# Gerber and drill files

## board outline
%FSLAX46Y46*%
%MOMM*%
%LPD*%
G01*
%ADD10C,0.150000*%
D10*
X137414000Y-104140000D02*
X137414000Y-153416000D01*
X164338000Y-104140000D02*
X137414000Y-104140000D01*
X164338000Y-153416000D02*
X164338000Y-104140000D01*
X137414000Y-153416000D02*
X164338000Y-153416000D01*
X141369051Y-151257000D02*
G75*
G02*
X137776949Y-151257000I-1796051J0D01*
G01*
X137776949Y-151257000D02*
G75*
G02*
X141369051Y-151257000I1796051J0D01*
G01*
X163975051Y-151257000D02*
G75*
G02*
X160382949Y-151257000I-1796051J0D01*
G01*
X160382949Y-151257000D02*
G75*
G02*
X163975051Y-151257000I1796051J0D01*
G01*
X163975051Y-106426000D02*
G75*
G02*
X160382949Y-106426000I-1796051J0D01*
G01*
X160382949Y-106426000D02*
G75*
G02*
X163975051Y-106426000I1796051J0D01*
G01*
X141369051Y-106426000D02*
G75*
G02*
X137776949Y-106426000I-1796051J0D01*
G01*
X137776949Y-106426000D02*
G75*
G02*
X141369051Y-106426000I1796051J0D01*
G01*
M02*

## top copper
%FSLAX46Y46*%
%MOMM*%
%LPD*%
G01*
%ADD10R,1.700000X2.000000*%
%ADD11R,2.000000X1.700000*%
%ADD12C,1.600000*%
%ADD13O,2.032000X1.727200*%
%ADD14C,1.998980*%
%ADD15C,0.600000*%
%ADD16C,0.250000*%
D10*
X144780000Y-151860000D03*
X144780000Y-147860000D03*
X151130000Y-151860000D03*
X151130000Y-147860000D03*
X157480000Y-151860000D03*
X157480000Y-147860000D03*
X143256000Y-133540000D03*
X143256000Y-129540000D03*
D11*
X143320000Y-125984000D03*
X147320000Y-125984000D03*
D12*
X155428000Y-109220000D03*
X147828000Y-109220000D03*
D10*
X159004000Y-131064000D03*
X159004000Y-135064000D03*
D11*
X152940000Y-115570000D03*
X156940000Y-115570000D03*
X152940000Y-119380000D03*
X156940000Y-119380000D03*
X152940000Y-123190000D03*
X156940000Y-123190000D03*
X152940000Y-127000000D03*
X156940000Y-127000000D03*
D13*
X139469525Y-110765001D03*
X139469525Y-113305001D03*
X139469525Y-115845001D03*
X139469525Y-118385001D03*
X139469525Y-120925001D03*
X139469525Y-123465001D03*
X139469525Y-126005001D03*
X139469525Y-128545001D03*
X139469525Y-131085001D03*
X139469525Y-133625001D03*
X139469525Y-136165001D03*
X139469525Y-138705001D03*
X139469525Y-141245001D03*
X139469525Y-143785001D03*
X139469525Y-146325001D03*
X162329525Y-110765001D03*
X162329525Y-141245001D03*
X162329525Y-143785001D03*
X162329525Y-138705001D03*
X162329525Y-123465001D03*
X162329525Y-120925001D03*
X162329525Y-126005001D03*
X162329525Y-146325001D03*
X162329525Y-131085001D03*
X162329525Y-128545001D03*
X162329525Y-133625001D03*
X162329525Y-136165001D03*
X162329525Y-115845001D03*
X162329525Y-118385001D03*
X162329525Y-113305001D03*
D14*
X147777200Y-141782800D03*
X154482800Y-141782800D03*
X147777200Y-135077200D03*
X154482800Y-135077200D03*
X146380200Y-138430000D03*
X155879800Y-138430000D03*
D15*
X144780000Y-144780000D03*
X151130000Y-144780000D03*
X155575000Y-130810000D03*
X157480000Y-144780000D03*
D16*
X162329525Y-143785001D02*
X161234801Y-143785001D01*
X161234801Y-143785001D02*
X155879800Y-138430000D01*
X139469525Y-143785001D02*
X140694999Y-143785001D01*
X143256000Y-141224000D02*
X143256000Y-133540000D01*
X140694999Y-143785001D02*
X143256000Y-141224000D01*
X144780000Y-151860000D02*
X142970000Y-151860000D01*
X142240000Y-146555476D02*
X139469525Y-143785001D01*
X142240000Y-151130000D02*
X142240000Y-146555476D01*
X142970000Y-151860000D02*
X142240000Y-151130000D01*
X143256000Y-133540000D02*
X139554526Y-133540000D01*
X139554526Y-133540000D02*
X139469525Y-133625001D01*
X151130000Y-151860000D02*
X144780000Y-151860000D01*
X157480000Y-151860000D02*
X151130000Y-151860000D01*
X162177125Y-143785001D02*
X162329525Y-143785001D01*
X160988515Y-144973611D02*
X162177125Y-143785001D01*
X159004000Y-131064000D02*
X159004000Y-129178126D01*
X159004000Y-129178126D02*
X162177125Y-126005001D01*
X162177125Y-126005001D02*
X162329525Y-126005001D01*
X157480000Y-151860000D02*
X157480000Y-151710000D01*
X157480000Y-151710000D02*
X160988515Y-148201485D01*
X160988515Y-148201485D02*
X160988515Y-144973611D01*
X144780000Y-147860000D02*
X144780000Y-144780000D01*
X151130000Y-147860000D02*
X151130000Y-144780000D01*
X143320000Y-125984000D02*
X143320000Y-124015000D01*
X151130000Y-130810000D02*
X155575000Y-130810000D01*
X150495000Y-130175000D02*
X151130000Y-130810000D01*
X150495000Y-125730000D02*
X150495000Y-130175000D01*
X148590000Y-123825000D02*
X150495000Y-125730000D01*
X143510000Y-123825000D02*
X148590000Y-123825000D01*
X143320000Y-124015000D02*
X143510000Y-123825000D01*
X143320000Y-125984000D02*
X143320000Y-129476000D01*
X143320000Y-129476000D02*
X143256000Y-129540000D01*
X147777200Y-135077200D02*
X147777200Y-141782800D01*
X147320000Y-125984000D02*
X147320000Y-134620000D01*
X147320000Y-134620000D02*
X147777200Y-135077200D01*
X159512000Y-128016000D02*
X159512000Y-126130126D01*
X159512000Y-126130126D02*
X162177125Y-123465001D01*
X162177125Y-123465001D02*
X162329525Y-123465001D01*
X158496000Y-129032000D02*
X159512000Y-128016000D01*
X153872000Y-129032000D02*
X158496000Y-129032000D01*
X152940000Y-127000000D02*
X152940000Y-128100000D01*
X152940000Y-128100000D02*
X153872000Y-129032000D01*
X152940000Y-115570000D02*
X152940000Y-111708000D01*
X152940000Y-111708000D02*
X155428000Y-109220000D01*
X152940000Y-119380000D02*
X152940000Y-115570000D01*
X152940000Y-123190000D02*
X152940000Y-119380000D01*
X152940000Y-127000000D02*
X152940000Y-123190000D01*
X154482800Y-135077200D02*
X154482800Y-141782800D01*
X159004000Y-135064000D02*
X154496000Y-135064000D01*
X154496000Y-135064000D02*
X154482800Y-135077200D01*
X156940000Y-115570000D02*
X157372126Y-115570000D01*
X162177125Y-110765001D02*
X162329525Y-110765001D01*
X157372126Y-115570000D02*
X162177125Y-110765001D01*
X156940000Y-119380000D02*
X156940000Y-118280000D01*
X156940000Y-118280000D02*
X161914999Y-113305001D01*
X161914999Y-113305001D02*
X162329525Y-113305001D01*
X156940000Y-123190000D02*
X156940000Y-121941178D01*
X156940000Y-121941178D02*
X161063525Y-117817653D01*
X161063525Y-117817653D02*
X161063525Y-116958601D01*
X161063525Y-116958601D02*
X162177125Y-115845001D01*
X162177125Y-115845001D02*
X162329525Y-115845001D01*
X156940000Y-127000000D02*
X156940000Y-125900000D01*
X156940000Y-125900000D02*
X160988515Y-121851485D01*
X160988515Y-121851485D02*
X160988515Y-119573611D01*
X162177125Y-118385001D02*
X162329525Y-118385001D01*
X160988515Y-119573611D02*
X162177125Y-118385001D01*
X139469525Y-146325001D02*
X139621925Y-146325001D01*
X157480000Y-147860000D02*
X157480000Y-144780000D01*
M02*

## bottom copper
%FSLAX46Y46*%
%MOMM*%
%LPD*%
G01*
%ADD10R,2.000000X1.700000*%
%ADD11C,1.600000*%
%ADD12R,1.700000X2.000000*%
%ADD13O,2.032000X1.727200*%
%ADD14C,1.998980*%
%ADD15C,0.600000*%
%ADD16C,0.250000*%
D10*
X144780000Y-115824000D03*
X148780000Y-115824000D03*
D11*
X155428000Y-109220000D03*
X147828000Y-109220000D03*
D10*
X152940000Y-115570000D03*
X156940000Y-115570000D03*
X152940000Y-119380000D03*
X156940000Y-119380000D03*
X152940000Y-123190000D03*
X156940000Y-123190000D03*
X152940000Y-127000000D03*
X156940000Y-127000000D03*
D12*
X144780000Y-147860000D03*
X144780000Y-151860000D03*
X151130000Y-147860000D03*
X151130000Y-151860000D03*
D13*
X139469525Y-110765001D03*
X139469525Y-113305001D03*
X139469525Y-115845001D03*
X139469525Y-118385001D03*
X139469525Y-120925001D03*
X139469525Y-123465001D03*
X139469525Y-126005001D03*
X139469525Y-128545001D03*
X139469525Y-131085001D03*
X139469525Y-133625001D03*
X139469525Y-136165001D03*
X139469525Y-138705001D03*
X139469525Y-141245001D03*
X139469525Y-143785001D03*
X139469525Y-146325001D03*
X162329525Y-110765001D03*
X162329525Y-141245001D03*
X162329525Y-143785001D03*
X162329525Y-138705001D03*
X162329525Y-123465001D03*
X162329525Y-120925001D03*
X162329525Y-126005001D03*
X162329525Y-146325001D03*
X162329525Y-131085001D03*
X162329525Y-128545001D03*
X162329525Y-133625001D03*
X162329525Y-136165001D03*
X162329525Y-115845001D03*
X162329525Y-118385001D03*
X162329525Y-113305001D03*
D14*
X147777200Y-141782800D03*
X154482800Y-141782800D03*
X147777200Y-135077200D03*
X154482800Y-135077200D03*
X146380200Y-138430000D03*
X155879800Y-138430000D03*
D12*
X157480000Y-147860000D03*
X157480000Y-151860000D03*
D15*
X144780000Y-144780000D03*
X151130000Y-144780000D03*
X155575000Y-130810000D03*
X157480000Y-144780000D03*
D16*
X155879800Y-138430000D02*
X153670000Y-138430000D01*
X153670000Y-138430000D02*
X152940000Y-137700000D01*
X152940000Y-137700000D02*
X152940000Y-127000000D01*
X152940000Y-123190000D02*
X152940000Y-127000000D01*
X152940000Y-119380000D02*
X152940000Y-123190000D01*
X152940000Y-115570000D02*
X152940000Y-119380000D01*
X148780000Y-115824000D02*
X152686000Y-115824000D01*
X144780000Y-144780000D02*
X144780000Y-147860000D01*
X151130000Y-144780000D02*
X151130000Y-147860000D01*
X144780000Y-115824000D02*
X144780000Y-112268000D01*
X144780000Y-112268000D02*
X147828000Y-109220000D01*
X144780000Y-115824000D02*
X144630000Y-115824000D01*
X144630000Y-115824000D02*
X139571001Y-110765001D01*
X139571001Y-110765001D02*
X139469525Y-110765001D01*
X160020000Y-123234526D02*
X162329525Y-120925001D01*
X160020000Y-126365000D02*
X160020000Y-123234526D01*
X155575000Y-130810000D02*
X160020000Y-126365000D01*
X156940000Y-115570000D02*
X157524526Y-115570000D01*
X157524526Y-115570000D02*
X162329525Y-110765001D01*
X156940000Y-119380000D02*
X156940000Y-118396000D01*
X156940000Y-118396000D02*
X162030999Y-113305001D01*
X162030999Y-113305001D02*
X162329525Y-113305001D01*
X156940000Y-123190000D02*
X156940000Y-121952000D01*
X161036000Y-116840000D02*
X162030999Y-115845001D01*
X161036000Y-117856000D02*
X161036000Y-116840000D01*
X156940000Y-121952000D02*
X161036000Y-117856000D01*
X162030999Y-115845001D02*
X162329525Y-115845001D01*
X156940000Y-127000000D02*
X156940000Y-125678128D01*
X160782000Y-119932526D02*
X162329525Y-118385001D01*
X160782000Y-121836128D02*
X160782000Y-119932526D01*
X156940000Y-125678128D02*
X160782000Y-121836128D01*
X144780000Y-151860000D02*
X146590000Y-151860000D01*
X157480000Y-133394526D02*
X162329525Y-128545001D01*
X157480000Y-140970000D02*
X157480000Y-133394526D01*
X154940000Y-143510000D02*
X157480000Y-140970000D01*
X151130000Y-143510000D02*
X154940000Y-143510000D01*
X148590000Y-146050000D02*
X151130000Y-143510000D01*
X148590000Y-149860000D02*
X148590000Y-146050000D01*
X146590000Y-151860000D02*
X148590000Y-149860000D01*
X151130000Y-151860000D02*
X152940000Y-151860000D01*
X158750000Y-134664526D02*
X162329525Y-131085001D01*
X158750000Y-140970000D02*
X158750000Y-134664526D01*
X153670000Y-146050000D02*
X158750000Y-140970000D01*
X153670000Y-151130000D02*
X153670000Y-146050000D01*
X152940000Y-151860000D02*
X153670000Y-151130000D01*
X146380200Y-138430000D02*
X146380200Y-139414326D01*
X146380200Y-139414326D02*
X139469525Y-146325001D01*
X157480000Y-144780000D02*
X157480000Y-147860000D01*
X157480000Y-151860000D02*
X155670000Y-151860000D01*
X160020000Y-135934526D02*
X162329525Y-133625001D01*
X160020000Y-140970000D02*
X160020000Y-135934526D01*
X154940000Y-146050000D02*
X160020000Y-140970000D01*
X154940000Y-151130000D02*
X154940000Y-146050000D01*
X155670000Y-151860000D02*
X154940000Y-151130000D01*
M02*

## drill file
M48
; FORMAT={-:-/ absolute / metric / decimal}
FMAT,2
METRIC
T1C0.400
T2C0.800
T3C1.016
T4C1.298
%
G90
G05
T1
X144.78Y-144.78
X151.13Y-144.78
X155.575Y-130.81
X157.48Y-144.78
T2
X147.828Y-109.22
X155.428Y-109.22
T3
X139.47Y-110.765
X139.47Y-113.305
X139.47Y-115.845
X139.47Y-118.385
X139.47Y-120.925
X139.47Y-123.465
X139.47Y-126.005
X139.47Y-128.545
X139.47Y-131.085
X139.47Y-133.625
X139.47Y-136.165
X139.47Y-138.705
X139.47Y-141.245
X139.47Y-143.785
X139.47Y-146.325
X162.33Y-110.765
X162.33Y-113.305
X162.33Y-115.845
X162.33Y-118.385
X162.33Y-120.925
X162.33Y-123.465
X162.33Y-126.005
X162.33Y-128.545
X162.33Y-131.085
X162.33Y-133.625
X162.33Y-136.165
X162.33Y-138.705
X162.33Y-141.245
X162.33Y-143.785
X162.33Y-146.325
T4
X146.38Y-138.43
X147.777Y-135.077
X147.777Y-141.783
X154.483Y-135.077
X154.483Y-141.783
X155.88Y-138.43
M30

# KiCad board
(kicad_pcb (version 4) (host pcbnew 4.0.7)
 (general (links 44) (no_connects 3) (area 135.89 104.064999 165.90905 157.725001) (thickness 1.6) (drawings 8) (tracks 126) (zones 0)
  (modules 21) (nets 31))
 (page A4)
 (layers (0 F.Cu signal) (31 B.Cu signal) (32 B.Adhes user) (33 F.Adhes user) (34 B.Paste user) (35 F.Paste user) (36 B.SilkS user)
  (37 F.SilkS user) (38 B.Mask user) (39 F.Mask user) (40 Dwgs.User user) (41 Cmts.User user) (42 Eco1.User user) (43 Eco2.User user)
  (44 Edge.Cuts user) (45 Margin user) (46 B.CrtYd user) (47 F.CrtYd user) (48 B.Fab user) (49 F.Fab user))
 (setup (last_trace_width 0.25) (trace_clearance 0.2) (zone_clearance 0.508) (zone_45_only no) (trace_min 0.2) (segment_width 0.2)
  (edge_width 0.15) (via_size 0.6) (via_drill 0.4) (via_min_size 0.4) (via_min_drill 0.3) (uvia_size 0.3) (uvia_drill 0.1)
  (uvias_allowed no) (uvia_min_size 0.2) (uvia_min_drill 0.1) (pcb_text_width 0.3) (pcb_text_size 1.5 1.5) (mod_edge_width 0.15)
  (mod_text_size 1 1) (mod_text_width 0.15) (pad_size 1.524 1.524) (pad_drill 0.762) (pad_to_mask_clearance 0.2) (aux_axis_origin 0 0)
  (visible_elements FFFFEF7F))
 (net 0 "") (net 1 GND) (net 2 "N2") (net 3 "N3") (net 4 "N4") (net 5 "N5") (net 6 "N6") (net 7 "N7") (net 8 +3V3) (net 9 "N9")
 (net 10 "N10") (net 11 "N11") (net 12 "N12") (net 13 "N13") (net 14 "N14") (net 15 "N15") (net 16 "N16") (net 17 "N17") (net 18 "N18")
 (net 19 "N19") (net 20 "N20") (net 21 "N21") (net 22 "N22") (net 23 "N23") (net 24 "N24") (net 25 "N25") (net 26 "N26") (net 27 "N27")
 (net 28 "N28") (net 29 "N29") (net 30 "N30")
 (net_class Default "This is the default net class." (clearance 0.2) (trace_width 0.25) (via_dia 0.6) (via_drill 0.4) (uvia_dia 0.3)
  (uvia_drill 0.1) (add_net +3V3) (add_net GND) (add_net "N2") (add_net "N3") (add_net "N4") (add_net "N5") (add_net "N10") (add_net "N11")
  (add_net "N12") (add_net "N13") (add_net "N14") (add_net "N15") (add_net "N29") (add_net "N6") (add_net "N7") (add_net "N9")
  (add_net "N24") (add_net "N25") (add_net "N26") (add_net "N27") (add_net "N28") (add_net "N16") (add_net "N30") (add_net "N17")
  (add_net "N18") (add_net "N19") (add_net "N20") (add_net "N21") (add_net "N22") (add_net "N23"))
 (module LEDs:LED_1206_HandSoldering (layer F.Cu) (at 144.78 149.86 90)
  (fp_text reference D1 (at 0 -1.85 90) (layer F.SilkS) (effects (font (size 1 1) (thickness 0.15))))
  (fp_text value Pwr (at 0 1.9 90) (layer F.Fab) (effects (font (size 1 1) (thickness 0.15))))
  (pad 1 smd rect (at -2 0 90) (size 2 1.7) (layers F.Cu F.Paste F.Mask) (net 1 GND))
  (pad 2 smd rect (at 2 0 90) (size 2 1.7) (layers F.Cu F.Paste F.Mask) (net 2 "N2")))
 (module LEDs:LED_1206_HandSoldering (layer F.Cu) (at 151.13 149.86 90)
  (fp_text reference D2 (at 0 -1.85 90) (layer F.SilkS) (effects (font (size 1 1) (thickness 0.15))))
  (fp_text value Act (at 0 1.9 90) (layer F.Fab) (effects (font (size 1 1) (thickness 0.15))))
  (pad 1 smd rect (at -2 0 90) (size 2 1.7) (layers F.Cu F.Paste F.Mask) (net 1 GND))
  (pad 2 smd rect (at 2 0 90) (size 2 1.7) (layers F.Cu F.Paste F.Mask) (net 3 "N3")))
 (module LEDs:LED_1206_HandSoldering (layer F.Cu) (at 157.48 149.86 90)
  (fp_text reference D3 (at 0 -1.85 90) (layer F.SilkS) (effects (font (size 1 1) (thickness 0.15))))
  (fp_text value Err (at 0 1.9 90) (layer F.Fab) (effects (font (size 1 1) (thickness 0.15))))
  (pad 1 smd rect (at -2 0 90) (size 2 1.7) (layers F.Cu F.Paste F.Mask) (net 1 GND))
  (pad 2 smd rect (at 2 0 90) (size 2 1.7) (layers F.Cu F.Paste F.Mask) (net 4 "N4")))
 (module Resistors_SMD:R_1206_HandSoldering (layer B.Cu) (at 146.78 115.824)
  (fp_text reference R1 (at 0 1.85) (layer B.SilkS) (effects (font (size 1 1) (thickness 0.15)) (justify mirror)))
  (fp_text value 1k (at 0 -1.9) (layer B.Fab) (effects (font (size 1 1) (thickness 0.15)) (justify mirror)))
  (pad 1 smd rect (at -2 0) (size 2 1.7) (layers B.Cu B.Paste B.Mask) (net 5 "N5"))
  (pad 2 smd rect (at 2 0) (size 2 1.7) (layers B.Cu B.Paste B.Mask) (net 1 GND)))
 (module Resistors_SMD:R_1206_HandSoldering (layer F.Cu) (at 143.256 131.54 90)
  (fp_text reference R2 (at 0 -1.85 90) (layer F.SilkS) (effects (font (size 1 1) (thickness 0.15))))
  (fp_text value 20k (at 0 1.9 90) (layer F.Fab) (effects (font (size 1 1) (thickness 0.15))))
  (pad 1 smd rect (at -2 0 90) (size 2 1.7) (layers F.Cu F.Paste F.Mask) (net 1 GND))
  (pad 2 smd rect (at 2 0 90) (size 2 1.7) (layers F.Cu F.Paste F.Mask) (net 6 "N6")))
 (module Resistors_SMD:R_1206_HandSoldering (layer F.Cu) (at 145.32 125.984)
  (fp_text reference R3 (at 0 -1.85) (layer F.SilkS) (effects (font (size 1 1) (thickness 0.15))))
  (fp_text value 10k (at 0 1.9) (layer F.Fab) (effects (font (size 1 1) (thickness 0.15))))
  (pad 1 smd rect (at -2 0) (size 2 1.7) (layers F.Cu F.Paste F.Mask) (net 6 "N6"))
  (pad 2 smd rect (at 2 0) (size 2 1.7) (layers F.Cu F.Paste F.Mask) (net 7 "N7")))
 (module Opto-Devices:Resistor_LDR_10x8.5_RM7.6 (layer F.Cu) (at 155.428 109.22 180)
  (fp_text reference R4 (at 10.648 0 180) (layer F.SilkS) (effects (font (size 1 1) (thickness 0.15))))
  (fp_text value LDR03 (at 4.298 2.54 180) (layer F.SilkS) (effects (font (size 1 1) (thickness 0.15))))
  (pad 1 thru_hole circle (at 0 0 180) (size 1.6 1.6) (drill 0.8) (layers *.Cu *.Mask) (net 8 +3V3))
  (pad 2 thru_hole circle (at 7.6 0 180) (size 1.6 1.6) (drill 0.8) (layers *.Cu *.Mask) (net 5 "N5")))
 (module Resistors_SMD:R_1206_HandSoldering (layer F.Cu) (at 159.004 133.064 270)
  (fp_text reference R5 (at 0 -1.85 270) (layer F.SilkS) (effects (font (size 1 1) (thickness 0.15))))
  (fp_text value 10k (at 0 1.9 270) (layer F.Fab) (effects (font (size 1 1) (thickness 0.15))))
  (pad 1 smd rect (at -2 0 270) (size 2 1.7) (layers F.Cu F.Paste F.Mask) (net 1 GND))
  (pad 2 smd rect (at 2 0 270) (size 2 1.7) (layers F.Cu F.Paste F.Mask) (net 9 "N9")))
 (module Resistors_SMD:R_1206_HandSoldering (layer F.Cu) (at 154.94 115.57)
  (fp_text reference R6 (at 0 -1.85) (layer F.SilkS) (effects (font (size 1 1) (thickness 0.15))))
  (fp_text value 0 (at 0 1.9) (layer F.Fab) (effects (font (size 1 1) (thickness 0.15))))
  (pad 1 smd rect (at -2 0) (size 2 1.7) (layers F.Cu F.Paste F.Mask) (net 8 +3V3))
  (pad 2 smd rect (at 2 0) (size 2 1.7) (layers F.Cu F.Paste F.Mask) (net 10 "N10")))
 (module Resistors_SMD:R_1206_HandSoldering (layer F.Cu) (at 154.94 119.38)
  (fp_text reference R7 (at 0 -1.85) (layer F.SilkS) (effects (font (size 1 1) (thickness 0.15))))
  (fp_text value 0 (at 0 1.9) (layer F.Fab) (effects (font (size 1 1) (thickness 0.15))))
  (pad 1 smd rect (at -2 0) (size 2 1.7) (layers F.Cu F.Paste F.Mask) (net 8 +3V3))
  (pad 2 smd rect (at 2 0) (size 2 1.7) (layers F.Cu F.Paste F.Mask) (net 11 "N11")))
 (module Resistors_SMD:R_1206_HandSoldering (layer F.Cu) (at 154.94 123.19)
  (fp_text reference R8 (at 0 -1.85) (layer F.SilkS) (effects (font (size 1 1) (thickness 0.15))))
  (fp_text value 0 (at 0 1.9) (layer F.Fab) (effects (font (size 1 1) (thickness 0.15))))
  (pad 1 smd rect (at -2 0) (size 2 1.7) (layers F.Cu F.Paste F.Mask) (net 8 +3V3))
  (pad 2 smd rect (at 2 0) (size 2 1.7) (layers F.Cu F.Paste F.Mask) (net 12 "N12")))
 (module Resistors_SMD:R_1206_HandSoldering (layer F.Cu) (at 154.94 127)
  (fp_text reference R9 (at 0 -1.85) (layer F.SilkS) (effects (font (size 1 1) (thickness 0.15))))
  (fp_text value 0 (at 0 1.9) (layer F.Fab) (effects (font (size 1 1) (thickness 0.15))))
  (pad 1 smd rect (at -2 0) (size 2 1.7) (layers F.Cu F.Paste F.Mask) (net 8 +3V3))
  (pad 2 smd rect (at 2 0) (size 2 1.7) (layers F.Cu F.Paste F.Mask) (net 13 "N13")))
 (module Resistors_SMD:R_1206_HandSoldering (layer B.Cu) (at 154.94 115.57)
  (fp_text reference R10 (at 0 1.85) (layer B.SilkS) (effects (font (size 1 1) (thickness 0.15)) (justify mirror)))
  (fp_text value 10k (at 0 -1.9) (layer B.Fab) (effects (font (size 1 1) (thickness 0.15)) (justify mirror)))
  (pad 1 smd rect (at -2 0) (size 2 1.7) (layers B.Cu B.Paste B.Mask) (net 1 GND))
  (pad 2 smd rect (at 2 0) (size 2 1.7) (layers B.Cu B.Paste B.Mask) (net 10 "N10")))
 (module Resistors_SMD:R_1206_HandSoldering (layer B.Cu) (at 154.94 119.38)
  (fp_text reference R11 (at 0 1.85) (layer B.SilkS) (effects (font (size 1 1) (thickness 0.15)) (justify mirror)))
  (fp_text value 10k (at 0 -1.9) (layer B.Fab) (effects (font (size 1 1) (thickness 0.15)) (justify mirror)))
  (pad 1 smd rect (at -2 0) (size 2 1.7) (layers B.Cu B.Paste B.Mask) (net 1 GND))
  (pad 2 smd rect (at 2 0) (size 2 1.7) (layers B.Cu B.Paste B.Mask) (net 11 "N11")))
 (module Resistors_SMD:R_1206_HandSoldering (layer B.Cu) (at 154.94 123.19)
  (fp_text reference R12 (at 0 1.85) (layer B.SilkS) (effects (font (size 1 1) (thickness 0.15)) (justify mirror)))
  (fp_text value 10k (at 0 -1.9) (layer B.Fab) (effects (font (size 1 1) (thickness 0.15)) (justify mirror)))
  (pad 1 smd rect (at -2 0) (size 2 1.7) (layers B.Cu B.Paste B.Mask) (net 1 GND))
  (pad 2 smd rect (at 2 0) (size 2 1.7) (layers B.Cu B.Paste B.Mask) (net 12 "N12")))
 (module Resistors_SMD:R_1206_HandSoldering (layer B.Cu) (at 154.94 127)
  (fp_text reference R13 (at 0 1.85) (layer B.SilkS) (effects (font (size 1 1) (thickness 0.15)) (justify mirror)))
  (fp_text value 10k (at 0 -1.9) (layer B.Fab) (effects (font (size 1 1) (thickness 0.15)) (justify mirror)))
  (pad 1 smd rect (at -2 0) (size 2 1.7) (layers B.Cu B.Paste B.Mask) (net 1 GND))
  (pad 2 smd rect (at 2 0) (size 2 1.7) (layers B.Cu B.Paste B.Mask) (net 13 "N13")))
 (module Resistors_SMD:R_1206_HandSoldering (layer B.Cu) (at 144.78 149.86 270)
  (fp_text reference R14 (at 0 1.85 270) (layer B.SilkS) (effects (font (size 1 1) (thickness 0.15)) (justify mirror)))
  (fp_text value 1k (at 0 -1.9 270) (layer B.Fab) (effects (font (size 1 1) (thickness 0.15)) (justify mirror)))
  (pad 1 smd rect (at -2 0 270) (size 2 1.7) (layers B.Cu B.Paste B.Mask) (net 2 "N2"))
  (pad 2 smd rect (at 2 0 270) (size 2 1.7) (layers B.Cu B.Paste B.Mask) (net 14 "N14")))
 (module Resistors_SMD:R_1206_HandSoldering (layer B.Cu) (at 151.13 149.86 270)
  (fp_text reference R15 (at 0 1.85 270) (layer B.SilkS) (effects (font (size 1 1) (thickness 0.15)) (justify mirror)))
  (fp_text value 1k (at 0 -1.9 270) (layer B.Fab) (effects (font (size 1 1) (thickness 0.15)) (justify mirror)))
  (pad 1 smd rect (at -2 0 270) (size 2 1.7) (layers B.Cu B.Paste B.Mask) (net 3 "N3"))
  (pad 2 smd rect (at 2 0 270) (size 2 1.7) (layers B.Cu B.Paste B.Mask) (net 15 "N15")))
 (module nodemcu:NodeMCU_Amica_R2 (layer F.Cu) (at 139.469525 110.765001)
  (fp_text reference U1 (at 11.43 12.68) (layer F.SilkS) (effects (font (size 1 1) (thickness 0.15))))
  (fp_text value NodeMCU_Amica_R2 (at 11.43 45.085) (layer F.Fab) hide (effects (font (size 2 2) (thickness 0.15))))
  (pad 1 thru_hole oval (at 0 0) (size 2.032 1.7272) (drill 1.016) (layers *.Cu *.Mask F.SilkS) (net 5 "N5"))
  (pad 2 thru_hole oval (at 0 2.54) (size 2.032 1.7272) (drill 1.016) (layers *.Cu *.Mask F.SilkS) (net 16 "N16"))
  (pad 3 thru_hole oval (at 0 5.08) (size 2.032 1.7272) (drill 1.016) (layers *.Cu *.Mask F.SilkS) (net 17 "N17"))
  (pad 4 thru_hole oval (at 0 7.62) (size 2.032 1.7272) (drill 1.016) (layers *.Cu *.Mask F.SilkS) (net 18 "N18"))
  (pad 5 thru_hole oval (at 0 10.16) (size 2.032 1.7272) (drill 1.016) (layers *.Cu *.Mask F.SilkS) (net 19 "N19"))
  (pad 6 thru_hole oval (at 0 12.7) (size 2.032 1.7272) (drill 1.016) (layers *.Cu *.Mask F.SilkS) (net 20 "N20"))
  (pad 7 thru_hole oval (at 0 15.24) (size 2.032 1.7272) (drill 1.016) (layers *.Cu *.Mask F.SilkS) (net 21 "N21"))
  (pad 8 thru_hole oval (at 0 17.78) (size 2.032 1.7272) (drill 1.016) (layers *.Cu *.Mask F.SilkS) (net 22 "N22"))
  (pad 9 thru_hole oval (at 0 20.32) (size 2.032 1.7272) (drill 1.016) (layers *.Cu *.Mask F.SilkS) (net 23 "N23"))
  (pad 10 thru_hole oval (at 0 22.86) (size 2.032 1.7272) (drill 1.016) (layers *.Cu *.Mask F.SilkS) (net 1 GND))
  (pad 11 thru_hole oval (at 0 25.4) (size 2.032 1.7272) (drill 1.016) (layers *.Cu *.Mask F.SilkS) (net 8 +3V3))
  (pad 12 thru_hole oval (at 0 27.94) (size 2.032 1.7272) (drill 1.016) (layers *.Cu *.Mask F.SilkS) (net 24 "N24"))
  (pad 13 thru_hole oval (at 0 30.48) (size 2.032 1.7272) (drill 1.016) (layers *.Cu *.Mask F.SilkS) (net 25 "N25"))
  (pad 14 thru_hole oval (at 0 33.02) (size 2.032 1.7272) (drill 1.016) (layers *.Cu *.Mask F.SilkS) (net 1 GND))
  (pad 15 thru_hole oval (at 0 35.56) (size 2.032 1.7272) (drill 1.016) (layers *.Cu *.Mask F.SilkS) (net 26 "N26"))
  (pad 30 thru_hole oval (at 22.86 0) (size 2.032 1.7272) (drill 1.016) (layers *.Cu *.Mask F.SilkS) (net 10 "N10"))
  (pad 18 thru_hole oval (at 22.86 30.48) (size 2.032 1.7272) (drill 1.016) (layers *.Cu *.Mask F.SilkS) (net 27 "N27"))
  (pad 17 thru_hole oval (at 22.86 33.02) (size 2.032 1.7272) (drill 1.016) (layers *.Cu *.Mask F.SilkS) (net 1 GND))
  (pad 19 thru_hole oval (at 22.86 27.94) (size 2.032 1.7272) (drill 1.016) (layers *.Cu *.Mask F.SilkS) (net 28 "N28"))
  (pad 25 thru_hole oval (at 22.86 12.7) (size 2.032 1.7272) (drill 1.016) (layers *.Cu *.Mask F.SilkS) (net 8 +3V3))
  (pad 26 thru_hole oval (at 22.86 10.16) (size 2.032 1.7272) (drill 1.016) (layers *.Cu *.Mask F.SilkS) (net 6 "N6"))
  (pad 24 thru_hole oval (at 22.86 15.24) (size 2.032 1.7272) (drill 1.016) (layers *.Cu *.Mask F.SilkS) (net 1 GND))
  (pad 16 thru_hole oval (at 22.86 35.56) (size 2.032 1.7272) (drill 1.016) (layers *.Cu *.Mask F.SilkS) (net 8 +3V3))
  (pad 22 thru_hole oval (at 22.86 20.32) (size 2.032 1.7272) (drill 1.016) (layers *.Cu *.Mask F.SilkS) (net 15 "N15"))
  (pad 23 thru_hole oval (at 22.86 17.78) (size 2.032 1.7272) (drill 1.016) (layers *.Cu *.Mask F.SilkS) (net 14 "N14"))
  (pad 21 thru_hole oval (at 22.86 22.86) (size 2.032 1.7272) (drill 1.016) (layers *.Cu *.Mask F.SilkS) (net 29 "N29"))
  (pad 20 thru_hole oval (at 22.86 25.4) (size 2.032 1.7272) (drill 1.016) (layers *.Cu *.Mask F.SilkS) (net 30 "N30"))
  (pad 28 thru_hole oval (at 22.86 5.08) (size 2.032 1.7272) (drill 1.016) (layers *.Cu *.Mask F.SilkS) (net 12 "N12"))
  (pad 27 thru_hole oval (at 22.86 7.62) (size 2.032 1.7272) (drill 1.016) (layers *.Cu *.Mask F.SilkS) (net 13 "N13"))
  (pad 29 thru_hole oval (at 22.86 2.54) (size 2.032 1.7272) (drill 1.016) (layers *.Cu *.Mask F.SilkS) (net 11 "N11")))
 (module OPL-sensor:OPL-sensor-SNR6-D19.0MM (layer F.Cu) (at 151.13 138.43 90)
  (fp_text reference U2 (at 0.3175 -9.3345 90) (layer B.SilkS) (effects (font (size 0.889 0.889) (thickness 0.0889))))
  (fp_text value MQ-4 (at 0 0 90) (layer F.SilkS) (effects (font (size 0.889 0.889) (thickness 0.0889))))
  (pad 1 thru_hole circle (at -3.3528 -3.3528 90) (size 1.99898 1.99898) (drill 1.29794) (layers *.Cu F.Paste F.SilkS F.Mask) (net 7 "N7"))
  (pad 2 thru_hole circle (at -3.3528 3.3528 90) (size 1.99898 1.99898) (drill 1.29794) (layers *.Cu F.Paste F.SilkS F.Mask) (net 9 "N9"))
  (pad 3 thru_hole circle (at 3.3528 -3.3528 90) (size 1.99898 1.99898) (drill 1.29794) (layers *.Cu F.Paste F.SilkS F.Mask) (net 7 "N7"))
  (pad 4 thru_hole circle (at 3.3528 3.3528 90) (size 1.99898 1.99898) (drill 1.29794) (layers *.Cu F.Paste F.SilkS F.Mask) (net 9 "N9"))
  (pad 5 thru_hole circle (at 0 -4.7498 90) (size 1.99898 1.99898) (drill 1.29794) (layers *.Cu F.Paste F.SilkS F.Mask) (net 26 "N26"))
  (pad 6 thru_hole circle (at 0 4.7498 90) (size 1.99898 1.99898) (drill 1.29794) (layers *.Cu F.Paste F.SilkS F.Mask) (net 1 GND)))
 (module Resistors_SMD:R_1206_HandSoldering (layer B.Cu) (at 157.48 149.86 270)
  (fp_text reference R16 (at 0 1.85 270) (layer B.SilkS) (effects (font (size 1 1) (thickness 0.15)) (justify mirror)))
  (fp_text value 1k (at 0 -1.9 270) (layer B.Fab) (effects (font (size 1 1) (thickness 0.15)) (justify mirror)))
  (pad 1 smd rect (at -2 0 270) (size 2 1.7) (layers B.Cu B.Paste B.Mask) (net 4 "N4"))
  (pad 2 smd rect (at 2 0 270) (size 2 1.7) (layers B.Cu B.Paste B.Mask) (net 29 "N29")))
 (gr_line (start 137.414 104.14) (end 137.414 153.416) (angle 90) (layer Edge.Cuts) (width 0.15))
 (gr_line (start 164.338 104.14) (end 137.414 104.14) (angle 90) (layer Edge.Cuts) (width 0.15))
 (gr_line (start 164.338 153.416) (end 164.338 104.14) (angle 90) (layer Edge.Cuts) (width 0.15))
 (gr_line (start 137.414 153.416) (end 164.338 153.416) (angle 90) (layer Edge.Cuts) (width 0.15))
 (gr_circle (center 139.573 151.257) (end 140.843 152.527) (layer Edge.Cuts) (width 0.15))
 (gr_circle (center 162.179 151.257) (end 163.449 152.527) (layer Edge.Cuts) (width 0.15))
 (gr_circle (center 162.179 106.426) (end 163.449 107.696) (layer Edge.Cuts) (width 0.15))
 (gr_circle (center 139.573 106.426) (end 140.843 107.696) (layer Edge.Cuts) (width 0.15))
 (segment (start 162.329525 143.785001) (end 161.234801 143.785001) (width 0.25) (layer F.Cu) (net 1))
 (segment (start 161.234801 143.785001) (end 155.8798 138.43) (width 0.25) (layer F.Cu) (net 1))
 (segment (start 139.469525 143.785001) (end 140.694999 143.785001) (width 0.25) (layer F.Cu) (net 1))
 (segment (start 143.256 141.224) (end 143.256 133.54) (width 0.25) (layer F.Cu) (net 1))
 (segment (start 140.694999 143.785001) (end 143.256 141.224) (width 0.25) (layer F.Cu) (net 1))
 (segment (start 144.78 151.86) (end 142.97 151.86) (width 0.25) (layer F.Cu) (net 1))
 (segment (start 142.24 146.555476) (end 139.469525 143.785001) (width 0.25) (layer F.Cu) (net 1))
 (segment (start 142.24 151.13) (end 142.24 146.555476) (width 0.25) (layer F.Cu) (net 1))
 (segment (start 142.97 151.86) (end 142.24 151.13) (width 0.25) (layer F.Cu) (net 1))
 (segment (start 155.8798 138.43) (end 153.67 138.43) (width 0.25) (layer B.Cu) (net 1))
 (segment (start 153.67 138.43) (end 152.94 137.7) (width 0.25) (layer B.Cu) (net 1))
 (segment (start 152.94 137.7) (end 152.94 127) (width 0.25) (layer B.Cu) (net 1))
 (segment (start 152.94 123.19) (end 152.94 127) (width 0.25) (layer B.Cu) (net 1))
 (segment (start 152.94 119.38) (end 152.94 123.19) (width 0.25) (layer B.Cu) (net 1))
 (segment (start 152.94 115.57) (end 152.94 119.38) (width 0.25) (layer B.Cu) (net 1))
 (segment (start 148.78 115.824) (end 152.686 115.824) (width 0.25) (layer B.Cu) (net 1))
 (segment (start 143.256 133.54) (end 139.554526 133.54) (width 0.25) (layer F.Cu) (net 1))
 (segment (start 139.554526 133.54) (end 139.469525 133.625001) (width 0.25) (layer F.Cu) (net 1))
 (segment (start 151.13 151.86) (end 144.78 151.86) (width 0.25) (layer F.Cu) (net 1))
 (segment (start 157.48 151.86) (end 151.13 151.86) (width 0.25) (layer F.Cu) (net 1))
 (segment (start 162.177125 143.785001) (end 162.329525 143.785001) (width 0.25) (layer F.Cu) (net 1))
 (segment (start 160.988515 144.973611) (end 162.177125 143.785001) (width 0.25) (layer F.Cu) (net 1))
 (segment (start 159.004 131.064) (end 159.004 129.178126) (width 0.25) (layer F.Cu) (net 1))
 (segment (start 159.004 129.178126) (end 162.177125 126.005001) (width 0.25) (layer F.Cu) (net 1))
 (segment (start 162.177125 126.005001) (end 162.329525 126.005001) (width 0.25) (layer F.Cu) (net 1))
 (segment (start 157.48 151.86) (end 157.48 151.71) (width 0.25) (layer F.Cu) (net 1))
 (segment (start 157.48 151.71) (end 160.988515 148.201485) (width 0.25) (layer F.Cu) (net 1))
 (segment (start 160.988515 148.201485) (end 160.988515 144.973611) (width 0.25) (layer F.Cu) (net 1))
 (segment (start 144.78 147.86) (end 144.78 144.78) (width 0.25) (layer F.Cu) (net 2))
 (segment (start 144.78 144.78) (end 144.78 147.86) (width 0.25) (layer B.Cu) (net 2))
 (via (at 144.78 144.78) (size 0.6) (drill 0.4) (layers F.Cu B.Cu) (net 2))
 (segment (start 151.13 147.86) (end 151.13 144.78) (width 0.25) (layer F.Cu) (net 3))
 (segment (start 151.13 144.78) (end 151.13 147.86) (width 0.25) (layer B.Cu) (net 3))
 (via (at 151.13 144.78) (size 0.6) (drill 0.4) (layers F.Cu B.Cu) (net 3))
 (segment (start 144.78 115.824) (end 144.78 112.268) (width 0.25) (layer B.Cu) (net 5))
 (segment (start 144.78 112.268) (end 147.828 109.22) (width 0.25) (layer B.Cu) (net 5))
 (segment (start 144.78 115.824) (end 144.63 115.824) (width 0.25) (layer B.Cu) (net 5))
 (segment (start 144.63 115.824) (end 139.571001 110.765001) (width 0.25) (layer B.Cu) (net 5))
 (segment (start 139.571001 110.765001) (end 139.469525 110.765001) (width 0.25) (layer B.Cu) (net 5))
 (segment (start 143.32 125.984) (end 143.32 124.015) (width 0.25) (layer F.Cu) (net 6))
 (segment (start 160.02 123.234526) (end 162.329525 120.925001) (width 0.25) (layer B.Cu) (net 6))
 (segment (start 160.02 126.365) (end 160.02 123.234526) (width 0.25) (layer B.Cu) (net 6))
 (segment (start 155.575 130.81) (end 160.02 126.365) (width 0.25) (layer B.Cu) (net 6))
 (via (at 155.575 130.81) (size 0.6) (drill 0.4) (layers F.Cu B.Cu) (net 6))
 (segment (start 151.13 130.81) (end 155.575 130.81) (width 0.25) (layer F.Cu) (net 6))
 (segment (start 150.495 130.175) (end 151.13 130.81) (width 0.25) (layer F.Cu) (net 6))
 (segment (start 150.495 125.73) (end 150.495 130.175) (width 0.25) (layer F.Cu) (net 6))
 (segment (start 148.59 123.825) (end 150.495 125.73) (width 0.25) (layer F.Cu) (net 6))
 (segment (start 143.51 123.825) (end 148.59 123.825) (width 0.25) (layer F.Cu) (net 6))
 (segment (start 143.32 124.015) (end 143.51 123.825) (width 0.25) (layer F.Cu) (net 6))
 (segment (start 143.32 125.984) (end 143.32 129.476) (width 0.25) (layer F.Cu) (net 6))
 (segment (start 143.32 129.476) (end 143.256 129.54) (width 0.25) (layer F.Cu) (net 6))
 (segment (start 147.7772 135.0772) (end 147.7772 141.7828) (width 0.25) (layer F.Cu) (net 7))
 (segment (start 147.32 125.984) (end 147.32 134.62) (width 0.25) (layer F.Cu) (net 7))
 (segment (start 147.32 134.62) (end 147.7772 135.0772) (width 0.25) (layer F.Cu) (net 7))
 (segment (start 159.512 128.016) (end 159.512 126.130126) (width 0.25) (layer F.Cu) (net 8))
 (segment (start 159.512 126.130126) (end 162.177125 123.465001) (width 0.25) (layer F.Cu) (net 8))
 (segment (start 162.177125 123.465001) (end 162.329525 123.465001) (width 0.25) (layer F.Cu) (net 8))
 (segment (start 158.496 129.032) (end 159.512 128.016) (width 0.25) (layer F.Cu) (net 8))
 (segment (start 153.872 129.032) (end 158.496 129.032) (width 0.25) (layer F.Cu) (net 8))
 (segment (start 152.94 127) (end 152.94 128.1) (width 0.25) (layer F.Cu) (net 8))
 (segment (start 152.94 128.1) (end 153.872 129.032) (width 0.25) (layer F.Cu) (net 8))
 (segment (start 152.94 115.57) (end 152.94 111.708) (width 0.25) (layer F.Cu) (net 8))
 (segment (start 152.94 111.708) (end 155.428 109.22) (width 0.25) (layer F.Cu) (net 8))
 (segment (start 152.94 119.38) (end 152.94 115.57) (width 0.25) (layer F.Cu) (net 8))
 (segment (start 152.94 123.19) (end 152.94 119.38) (width 0.25) (layer F.Cu) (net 8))
 (segment (start 152.94 127) (end 152.94 123.19) (width 0.25) (layer F.Cu) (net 8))
 (segment (start 154.4828 135.0772) (end 154.4828 141.7828) (width 0.25) (layer F.Cu) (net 9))
 (segment (start 159.004 135.064) (end 154.496 135.064) (width 0.25) (layer F.Cu) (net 9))
 (segment (start 154.496 135.064) (end 154.4828 135.0772) (width 0.25) (layer F.Cu) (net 9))
 (segment (start 156.94 115.57) (end 157.524526 115.57) (width 0.25) (layer B.Cu) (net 10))
 (segment (start 157.524526 115.57) (end 162.329525 110.765001) (width 0.25) (layer B.Cu) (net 10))
 (segment (start 156.94 115.57) (end 157.372126 115.57) (width 0.25) (layer F.Cu) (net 10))
 (segment (start 162.177125 110.765001) (end 162.329525 110.765001) (width 0.25) (layer F.Cu) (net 10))
 (segment (start 157.372126 115.57) (end 162.177125 110.765001) (width 0.25) (layer F.Cu) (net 10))
 (segment (start 156.94 119.38) (end 156.94 118.396) (width 0.25) (layer B.Cu) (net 11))
 (segment (start 156.94 118.396) (end 162.030999 113.305001) (width 0.25) (layer B.Cu) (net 11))
 (segment (start 162.030999 113.305001) (end 162.329525 113.305001) (width 0.25) (layer B.Cu) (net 11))
 (segment (start 156.94 119.38) (end 156.94 118.28) (width 0.25) (layer F.Cu) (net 11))
 (segment (start 156.94 118.28) (end 161.914999 113.305001) (width 0.25) (layer F.Cu) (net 11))
 (segment (start 161.914999 113.305001) (end 162.329525 113.305001) (width 0.25) (layer F.Cu) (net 11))
 (segment (start 156.94 123.19) (end 156.94 121.952) (width 0.25) (layer B.Cu) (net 12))
 (segment (start 161.036 116.84) (end 162.030999 115.845001) (width 0.25) (layer B.Cu) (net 12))
 (segment (start 161.036 117.856) (end 161.036 116.84) (width 0.25) (layer B.Cu) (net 12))
 (segment (start 156.94 121.952) (end 161.036 117.856) (width 0.25) (layer B.Cu) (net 12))
 (segment (start 162.030999 115.845001) (end 162.329525 115.845001) (width 0.25) (layer B.Cu) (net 12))
 (segment (start 156.94 123.19) (end 156.94 121.941178) (width 0.25) (layer F.Cu) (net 12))
 (segment (start 156.94 121.941178) (end 161.063525 117.817653) (width 0.25) (layer F.Cu) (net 12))
 (segment (start 161.063525 117.817653) (end 161.063525 116.958601) (width 0.25) (layer F.Cu) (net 12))
 (segment (start 161.063525 116.958601) (end 162.177125 115.845001) (width 0.25) (layer F.Cu) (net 12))
 (segment (start 162.177125 115.845001) (end 162.329525 115.845001) (width 0.25) (layer F.Cu) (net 12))
 (segment (start 156.94 127) (end 156.94 125.678128) (width 0.25) (layer B.Cu) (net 13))
 (segment (start 160.782 119.932526) (end 162.329525 118.385001) (width 0.25) (layer B.Cu) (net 13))
 (segment (start 160.782 121.836128) (end 160.782 119.932526) (width 0.25) (layer B.Cu) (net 13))
 (segment (start 156.94 125.678128) (end 160.782 121.836128) (width 0.25) (layer B.Cu) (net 13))
 (segment (start 156.94 127) (end 156.94 125.9) (width 0.25) (layer F.Cu) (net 13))
 (segment (start 156.94 125.9) (end 160.988515 121.851485) (width 0.25) (layer F.Cu) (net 13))
 (segment (start 160.988515 121.851485) (end 160.988515 119.573611) (width 0.25) (layer F.Cu) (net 13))
 (segment (start 162.177125 118.385001) (end 162.329525 118.385001) (width 0.25) (layer F.Cu) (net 13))
 (segment (start 160.988515 119.573611) (end 162.177125 118.385001) (width 0.25) (layer F.Cu) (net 13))
 (segment (start 144.78 151.86) (end 146.59 151.86) (width 0.25) (layer B.Cu) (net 14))
 (segment (start 157.48 133.394526) (end 162.329525 128.545001) (width 0.25) (layer B.Cu) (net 14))
 (segment (start 157.48 140.97) (end 157.48 133.394526) (width 0.25) (layer B.Cu) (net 14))
 (segment (start 154.94 143.51) (end 157.48 140.97) (width 0.25) (layer B.Cu) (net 14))
 (segment (start 151.13 143.51) (end 154.94 143.51) (width 0.25) (layer B.Cu) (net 14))
 (segment (start 148.59 146.05) (end 151.13 143.51) (width 0.25) (layer B.Cu) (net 14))
 (segment (start 148.59 149.86) (end 148.59 146.05) (width 0.25) (layer B.Cu) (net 14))
 (segment (start 146.59 151.86) (end 148.59 149.86) (width 0.25) (layer B.Cu) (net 14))
 (segment (start 151.13 151.86) (end 152.94 151.86) (width 0.25) (layer B.Cu) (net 15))
 (segment (start 158.75 134.664526) (end 162.329525 131.085001) (width 0.25) (layer B.Cu) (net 15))
 (segment (start 158.75 140.97) (end 158.75 134.664526) (width 0.25) (layer B.Cu) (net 15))
 (segment (start 153.67 146.05) (end 158.75 140.97) (width 0.25) (layer B.Cu) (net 15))
 (segment (start 153.67 151.13) (end 153.67 146.05) (width 0.25) (layer B.Cu) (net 15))
 (segment (start 152.94 151.86) (end 153.67 151.13) (width 0.25) (layer B.Cu) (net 15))
 (segment (start 146.3802 138.43) (end 146.3802 139.414326) (width 0.25) (layer B.Cu) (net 26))
 (segment (start 146.3802 139.414326) (end 139.469525 146.325001) (width 0.25) (layer B.Cu) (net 26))
 (segment (start 139.469525 146.325001) (end 139.621925 146.325001) (width 0.25) (layer F.Cu) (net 26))
 (segment (start 157.48 147.86) (end 157.48 144.78) (width 0.25) (layer F.Cu) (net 4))
 (segment (start 157.48 144.78) (end 157.48 147.86) (width 0.25) (layer B.Cu) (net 4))
 (via (at 157.48 144.78) (size 0.6) (drill 0.4) (layers F.Cu B.Cu) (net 4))
 (segment (start 157.48 151.86) (end 155.67 151.86) (width 0.25) (layer B.Cu) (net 29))
 (segment (start 160.02 135.934526) (end 162.329525 133.625001) (width 0.25) (layer B.Cu) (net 29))
 (segment (start 160.02 140.97) (end 160.02 135.934526) (width 0.25) (layer B.Cu) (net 29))
 (segment (start 154.94 146.05) (end 160.02 140.97) (width 0.25) (layer B.Cu) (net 29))
 (segment (start 154.94 151.13) (end 154.94 146.05) (width 0.25) (layer B.Cu) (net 29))
 (segment (start 155.67 151.86) (end 154.94 151.13) (width 0.25) (layer B.Cu) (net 29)))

